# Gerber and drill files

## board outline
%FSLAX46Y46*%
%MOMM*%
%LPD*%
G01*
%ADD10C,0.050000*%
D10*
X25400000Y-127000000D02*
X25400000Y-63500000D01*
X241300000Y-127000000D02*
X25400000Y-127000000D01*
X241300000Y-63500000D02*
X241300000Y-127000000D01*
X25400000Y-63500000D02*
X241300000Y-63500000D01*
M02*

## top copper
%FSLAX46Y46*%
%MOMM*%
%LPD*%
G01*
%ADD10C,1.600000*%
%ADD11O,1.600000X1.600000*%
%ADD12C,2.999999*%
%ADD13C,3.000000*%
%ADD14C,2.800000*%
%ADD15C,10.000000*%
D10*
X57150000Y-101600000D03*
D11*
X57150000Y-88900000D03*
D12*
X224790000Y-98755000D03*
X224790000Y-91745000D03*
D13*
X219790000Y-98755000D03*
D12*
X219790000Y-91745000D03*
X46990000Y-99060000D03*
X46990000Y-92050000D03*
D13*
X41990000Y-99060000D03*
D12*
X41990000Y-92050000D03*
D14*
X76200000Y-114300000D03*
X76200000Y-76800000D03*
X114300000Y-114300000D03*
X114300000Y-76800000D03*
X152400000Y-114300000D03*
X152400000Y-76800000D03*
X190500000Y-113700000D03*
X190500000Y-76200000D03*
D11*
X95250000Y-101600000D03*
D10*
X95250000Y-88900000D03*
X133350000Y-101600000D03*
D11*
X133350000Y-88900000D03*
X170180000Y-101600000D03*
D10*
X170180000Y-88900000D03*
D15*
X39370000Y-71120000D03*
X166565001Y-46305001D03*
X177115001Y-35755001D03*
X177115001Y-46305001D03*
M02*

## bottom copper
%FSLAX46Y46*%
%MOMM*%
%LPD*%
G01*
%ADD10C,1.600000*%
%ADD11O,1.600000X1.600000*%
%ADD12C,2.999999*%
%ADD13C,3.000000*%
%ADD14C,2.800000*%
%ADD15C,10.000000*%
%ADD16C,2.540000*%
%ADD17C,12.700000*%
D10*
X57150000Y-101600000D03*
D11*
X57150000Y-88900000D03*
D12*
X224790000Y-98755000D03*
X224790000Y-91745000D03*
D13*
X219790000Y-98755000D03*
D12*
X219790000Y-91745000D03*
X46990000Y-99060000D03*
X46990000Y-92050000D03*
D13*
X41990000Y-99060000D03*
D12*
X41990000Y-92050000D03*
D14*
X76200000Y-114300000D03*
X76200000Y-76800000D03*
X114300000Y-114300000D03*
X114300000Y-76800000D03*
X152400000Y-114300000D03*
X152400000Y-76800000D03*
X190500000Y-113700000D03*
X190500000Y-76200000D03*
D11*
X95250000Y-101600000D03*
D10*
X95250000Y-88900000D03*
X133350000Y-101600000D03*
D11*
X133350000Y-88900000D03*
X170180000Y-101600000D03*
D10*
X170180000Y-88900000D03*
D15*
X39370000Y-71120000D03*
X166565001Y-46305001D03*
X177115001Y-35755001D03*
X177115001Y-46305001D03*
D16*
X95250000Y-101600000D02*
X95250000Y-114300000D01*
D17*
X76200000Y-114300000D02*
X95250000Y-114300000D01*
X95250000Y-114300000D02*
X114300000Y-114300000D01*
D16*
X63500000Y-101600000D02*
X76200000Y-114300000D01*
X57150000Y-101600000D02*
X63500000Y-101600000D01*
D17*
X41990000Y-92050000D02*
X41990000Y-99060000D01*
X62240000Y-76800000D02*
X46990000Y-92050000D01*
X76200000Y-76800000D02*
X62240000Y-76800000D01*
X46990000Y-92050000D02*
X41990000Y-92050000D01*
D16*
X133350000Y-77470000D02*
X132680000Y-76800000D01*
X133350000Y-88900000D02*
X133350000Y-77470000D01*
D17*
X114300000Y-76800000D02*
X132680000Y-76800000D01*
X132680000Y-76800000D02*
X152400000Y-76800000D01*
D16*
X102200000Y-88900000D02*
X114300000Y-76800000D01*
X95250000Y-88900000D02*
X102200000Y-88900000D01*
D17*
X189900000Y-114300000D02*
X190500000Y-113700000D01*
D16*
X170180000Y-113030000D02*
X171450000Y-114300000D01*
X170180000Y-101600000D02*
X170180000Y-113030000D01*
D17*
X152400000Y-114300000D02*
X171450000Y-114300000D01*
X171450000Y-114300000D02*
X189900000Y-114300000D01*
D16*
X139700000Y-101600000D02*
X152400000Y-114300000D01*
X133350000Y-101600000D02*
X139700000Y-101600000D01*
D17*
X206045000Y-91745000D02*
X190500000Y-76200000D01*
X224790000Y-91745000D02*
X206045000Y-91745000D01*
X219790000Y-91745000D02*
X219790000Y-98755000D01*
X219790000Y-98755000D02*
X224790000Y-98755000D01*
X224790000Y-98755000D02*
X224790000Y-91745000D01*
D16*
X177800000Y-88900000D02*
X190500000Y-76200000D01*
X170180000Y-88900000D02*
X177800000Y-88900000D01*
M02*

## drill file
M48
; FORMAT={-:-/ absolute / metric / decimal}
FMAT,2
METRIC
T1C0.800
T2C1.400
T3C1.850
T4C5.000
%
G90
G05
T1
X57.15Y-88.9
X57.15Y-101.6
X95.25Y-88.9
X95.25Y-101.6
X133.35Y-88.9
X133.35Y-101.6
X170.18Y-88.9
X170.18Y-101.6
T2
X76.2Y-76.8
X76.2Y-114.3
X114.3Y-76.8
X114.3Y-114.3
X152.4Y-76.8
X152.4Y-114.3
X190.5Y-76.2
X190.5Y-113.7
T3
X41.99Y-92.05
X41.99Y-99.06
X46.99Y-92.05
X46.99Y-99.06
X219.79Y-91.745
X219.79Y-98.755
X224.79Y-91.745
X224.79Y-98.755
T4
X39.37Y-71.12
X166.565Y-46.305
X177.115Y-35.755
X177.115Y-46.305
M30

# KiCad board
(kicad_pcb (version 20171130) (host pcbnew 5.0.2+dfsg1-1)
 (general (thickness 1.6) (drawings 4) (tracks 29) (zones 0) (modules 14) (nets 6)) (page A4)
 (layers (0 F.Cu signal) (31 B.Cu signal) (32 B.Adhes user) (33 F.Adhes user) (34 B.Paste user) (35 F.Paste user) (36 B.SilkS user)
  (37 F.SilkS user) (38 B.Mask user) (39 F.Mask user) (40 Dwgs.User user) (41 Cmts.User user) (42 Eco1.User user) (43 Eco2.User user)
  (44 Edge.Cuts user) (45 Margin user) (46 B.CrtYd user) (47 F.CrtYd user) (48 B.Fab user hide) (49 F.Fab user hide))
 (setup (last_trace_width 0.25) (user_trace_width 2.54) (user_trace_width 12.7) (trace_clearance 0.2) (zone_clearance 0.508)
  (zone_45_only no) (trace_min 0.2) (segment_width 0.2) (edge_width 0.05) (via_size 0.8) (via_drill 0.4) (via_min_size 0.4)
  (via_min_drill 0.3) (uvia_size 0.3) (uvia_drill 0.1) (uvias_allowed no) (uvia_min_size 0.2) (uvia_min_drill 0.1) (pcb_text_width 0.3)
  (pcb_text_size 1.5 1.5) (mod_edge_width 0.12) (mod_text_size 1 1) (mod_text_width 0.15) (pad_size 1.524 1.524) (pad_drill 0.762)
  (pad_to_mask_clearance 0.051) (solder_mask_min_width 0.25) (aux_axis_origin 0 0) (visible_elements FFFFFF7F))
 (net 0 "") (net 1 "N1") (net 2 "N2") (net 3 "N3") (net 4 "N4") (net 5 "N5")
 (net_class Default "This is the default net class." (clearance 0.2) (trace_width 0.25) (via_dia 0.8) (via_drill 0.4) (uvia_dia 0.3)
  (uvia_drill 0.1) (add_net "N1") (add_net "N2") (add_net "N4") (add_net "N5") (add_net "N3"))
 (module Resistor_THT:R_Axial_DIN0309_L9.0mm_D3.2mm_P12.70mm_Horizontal (layer F.Cu) (at 57.15 101.6 90)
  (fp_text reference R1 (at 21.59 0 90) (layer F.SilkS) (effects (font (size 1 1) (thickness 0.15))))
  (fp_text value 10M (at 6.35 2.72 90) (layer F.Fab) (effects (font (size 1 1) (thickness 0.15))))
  (pad 1 thru_hole circle (at 0 0 90) (size 1.6 1.6) (drill 0.8) (layers *.Cu *.Mask) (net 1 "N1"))
  (pad 2 thru_hole oval (at 12.7 0 90) (size 1.6 1.6) (drill 0.8) (layers *.Cu *.Mask) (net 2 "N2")))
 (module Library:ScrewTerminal (layer F.Cu) (at 222.29 95.25)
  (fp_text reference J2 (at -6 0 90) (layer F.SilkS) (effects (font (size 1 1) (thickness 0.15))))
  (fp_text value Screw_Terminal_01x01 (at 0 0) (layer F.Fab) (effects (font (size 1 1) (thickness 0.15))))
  (pad 1 thru_hole circle (at 2.5 3.505) (size 2.999999 2.999999) (drill 1.85) (layers *.Cu *.Mask) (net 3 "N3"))
  (pad 1 thru_hole circle (at 2.5 -3.505) (size 2.999999 2.999999) (drill 1.85) (layers *.Cu *.Mask) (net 3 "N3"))
  (pad 1 thru_hole circle (at -2.5 3.505) (size 3 3) (drill 1.85) (layers *.Cu *.Mask) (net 3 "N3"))
  (pad 1 thru_hole circle (at -2.5 -3.505) (size 2.999999 2.999999) (drill 1.85) (layers *.Cu *.Mask) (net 3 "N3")))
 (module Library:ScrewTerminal (layer F.Cu) (at 44.49 95.555)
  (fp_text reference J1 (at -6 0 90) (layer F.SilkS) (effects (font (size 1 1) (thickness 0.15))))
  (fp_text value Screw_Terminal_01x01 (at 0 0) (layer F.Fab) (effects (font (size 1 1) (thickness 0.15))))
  (pad 1 thru_hole circle (at 2.5 3.505) (size 2.999999 2.999999) (drill 1.85) (layers *.Cu *.Mask) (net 2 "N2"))
  (pad 1 thru_hole circle (at 2.5 -3.505) (size 2.999999 2.999999) (drill 1.85) (layers *.Cu *.Mask) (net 2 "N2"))
  (pad 1 thru_hole circle (at -2.5 3.505) (size 3 3) (drill 1.85) (layers *.Cu *.Mask) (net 2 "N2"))
  (pad 1 thru_hole circle (at -2.5 -3.505) (size 2.999999 2.999999) (drill 1.85) (layers *.Cu *.Mask) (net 2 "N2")))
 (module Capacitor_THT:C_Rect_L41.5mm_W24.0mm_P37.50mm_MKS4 (layer F.Cu) (at 76.2 114.3 90)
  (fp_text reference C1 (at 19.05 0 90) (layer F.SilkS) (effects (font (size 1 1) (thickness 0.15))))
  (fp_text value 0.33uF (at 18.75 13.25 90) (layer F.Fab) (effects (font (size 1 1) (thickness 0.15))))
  (pad 1 thru_hole circle (at 0 0 90) (size 2.8 2.8) (drill 1.4) (layers *.Cu *.Mask) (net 1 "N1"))
  (pad 2 thru_hole circle (at 37.5 0 90) (size 2.8 2.8) (drill 1.4) (layers *.Cu *.Mask) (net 2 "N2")))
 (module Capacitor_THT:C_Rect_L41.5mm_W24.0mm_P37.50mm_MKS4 (layer F.Cu) (at 114.3 76.8 270)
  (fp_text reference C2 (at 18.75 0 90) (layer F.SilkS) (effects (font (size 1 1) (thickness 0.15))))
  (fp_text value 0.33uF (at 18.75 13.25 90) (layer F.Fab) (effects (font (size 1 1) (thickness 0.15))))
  (pad 2 thru_hole circle (at 37.5 0 270) (size 2.8 2.8) (drill 1.4) (layers *.Cu *.Mask) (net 1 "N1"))
  (pad 1 thru_hole circle (at 0 0 270) (size 2.8 2.8) (drill 1.4) (layers *.Cu *.Mask) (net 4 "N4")))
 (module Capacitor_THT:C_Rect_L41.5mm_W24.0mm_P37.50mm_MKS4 (layer F.Cu) (at 152.4 114.3 90)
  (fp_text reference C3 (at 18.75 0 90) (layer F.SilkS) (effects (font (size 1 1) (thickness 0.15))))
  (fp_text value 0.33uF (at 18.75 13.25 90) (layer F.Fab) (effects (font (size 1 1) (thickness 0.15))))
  (pad 1 thru_hole circle (at 0 0 90) (size 2.8 2.8) (drill 1.4) (layers *.Cu *.Mask) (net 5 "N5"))
  (pad 2 thru_hole circle (at 37.5 0 90) (size 2.8 2.8) (drill 1.4) (layers *.Cu *.Mask) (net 4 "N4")))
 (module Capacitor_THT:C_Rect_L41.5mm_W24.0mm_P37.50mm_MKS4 (layer F.Cu) (at 190.5 76.2 270)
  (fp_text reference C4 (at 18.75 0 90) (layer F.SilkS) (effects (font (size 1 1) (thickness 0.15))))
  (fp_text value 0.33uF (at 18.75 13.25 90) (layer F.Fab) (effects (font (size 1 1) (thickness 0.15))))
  (pad 2 thru_hole circle (at 37.5 0 270) (size 2.8 2.8) (drill 1.4) (layers *.Cu *.Mask) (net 5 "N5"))
  (pad 1 thru_hole circle (at 0 0 270) (size 2.8 2.8) (drill 1.4) (layers *.Cu *.Mask) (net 3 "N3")))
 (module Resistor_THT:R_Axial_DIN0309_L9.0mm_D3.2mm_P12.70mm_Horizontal (layer F.Cu) (at 95.25 88.9 270)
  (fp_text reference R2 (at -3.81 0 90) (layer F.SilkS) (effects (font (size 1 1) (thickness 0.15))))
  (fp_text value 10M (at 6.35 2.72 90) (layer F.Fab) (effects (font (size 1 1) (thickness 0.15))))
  (pad 2 thru_hole oval (at 12.7 0 270) (size 1.6 1.6) (drill 0.8) (layers *.Cu *.Mask) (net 1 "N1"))
  (pad 1 thru_hole circle (at 0 0 270) (size 1.6 1.6) (drill 0.8) (layers *.Cu *.Mask) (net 4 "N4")))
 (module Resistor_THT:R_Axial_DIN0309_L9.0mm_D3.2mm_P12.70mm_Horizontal (layer F.Cu) (at 133.35 101.6 90)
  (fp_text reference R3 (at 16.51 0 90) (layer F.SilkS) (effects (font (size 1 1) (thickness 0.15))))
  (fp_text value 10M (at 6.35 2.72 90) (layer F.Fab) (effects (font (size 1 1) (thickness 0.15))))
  (pad 1 thru_hole circle (at 0 0 90) (size 1.6 1.6) (drill 0.8) (layers *.Cu *.Mask) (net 5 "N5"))
  (pad 2 thru_hole oval (at 12.7 0 90) (size 1.6 1.6) (drill 0.8) (layers *.Cu *.Mask) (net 4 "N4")))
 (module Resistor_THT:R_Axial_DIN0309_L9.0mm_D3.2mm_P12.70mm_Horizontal (layer F.Cu) (at 170.18 88.9 270)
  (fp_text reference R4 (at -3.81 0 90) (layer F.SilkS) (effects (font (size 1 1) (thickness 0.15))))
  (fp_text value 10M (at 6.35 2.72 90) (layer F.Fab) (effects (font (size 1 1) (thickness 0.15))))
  (pad 2 thru_hole oval (at 12.7 0 270) (size 1.6 1.6) (drill 0.8) (layers *.Cu *.Mask) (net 5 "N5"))
  (pad 1 thru_hole circle (at 0 0 270) (size 1.6 1.6) (drill 0.8) (layers *.Cu *.Mask) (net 3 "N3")))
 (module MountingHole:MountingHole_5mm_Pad (layer F.Cu) (at 39.37 71.12)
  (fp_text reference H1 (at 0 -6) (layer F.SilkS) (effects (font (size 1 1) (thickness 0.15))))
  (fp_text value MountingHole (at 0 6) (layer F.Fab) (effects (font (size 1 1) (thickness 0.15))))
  (pad 1 thru_hole circle (at 0 0) (size 10 10) (drill 5) (layers *.Cu *.Mask)))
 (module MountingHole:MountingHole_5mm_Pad (layer F.Cu) (at 166.565001 46.305001)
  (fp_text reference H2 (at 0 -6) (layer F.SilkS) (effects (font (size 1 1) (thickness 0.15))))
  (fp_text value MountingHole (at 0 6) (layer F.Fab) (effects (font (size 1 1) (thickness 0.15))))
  (pad 1 thru_hole circle (at 0 0) (size 10 10) (drill 5) (layers *.Cu *.Mask)))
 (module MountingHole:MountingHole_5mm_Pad (layer F.Cu) (at 177.115001 35.755001)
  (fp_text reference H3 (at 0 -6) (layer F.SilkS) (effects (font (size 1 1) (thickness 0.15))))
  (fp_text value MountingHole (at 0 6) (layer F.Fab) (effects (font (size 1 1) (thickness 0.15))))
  (pad 1 thru_hole circle (at 0 0) (size 10 10) (drill 5) (layers *.Cu *.Mask)))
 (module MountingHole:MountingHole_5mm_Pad (layer F.Cu) (at 177.115001 46.305001)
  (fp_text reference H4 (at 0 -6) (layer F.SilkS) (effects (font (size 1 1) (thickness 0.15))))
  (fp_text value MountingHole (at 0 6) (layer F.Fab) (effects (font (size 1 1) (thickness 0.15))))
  (pad 1 thru_hole circle (at 0 0) (size 10 10) (drill 5) (layers *.Cu *.Mask)))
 (gr_line (start 25.4 127) (end 25.4 63.5) (layer Edge.Cuts) (width 0.05))
 (gr_line (start 241.3 127) (end 25.4 127) (layer Edge.Cuts) (width 0.05))
 (gr_line (start 241.3 63.5) (end 241.3 127) (layer Edge.Cuts) (width 0.05))
 (gr_line (start 25.4 63.5) (end 241.3 63.5) (layer Edge.Cuts) (width 0.05))
 (segment (start 95.25 101.6) (end 95.25 114.3) (width 2.54) (layer B.Cu) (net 1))
 (segment (start 76.2 114.3) (end 95.25 114.3) (width 12.7) (layer B.Cu) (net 1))
 (segment (start 95.25 114.3) (end 114.3 114.3) (width 12.7) (layer B.Cu) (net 1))
 (segment (start 63.5 101.6) (end 76.2 114.3) (width 2.54) (layer B.Cu) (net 1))
 (segment (start 57.15 101.6) (end 63.5 101.6) (width 2.54) (layer B.Cu) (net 1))
 (segment (start 41.99 92.05) (end 41.99 99.06) (width 12.7) (layer B.Cu) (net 2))
 (segment (start 62.24 76.8) (end 46.99 92.05) (width 12.7) (layer B.Cu) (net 2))
 (segment (start 76.2 76.8) (end 62.24 76.8) (width 12.7) (layer B.Cu) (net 2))
 (segment (start 46.99 92.05) (end 41.99 92.05) (width 12.7) (layer B.Cu) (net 2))
 (segment (start 133.35 77.47) (end 132.68 76.8) (width 2.54) (layer B.Cu) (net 4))
 (segment (start 133.35 88.9) (end 133.35 77.47) (width 2.54) (layer B.Cu) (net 4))
 (segment (start 114.3 76.8) (end 132.68 76.8) (width 12.7) (layer B.Cu) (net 4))
 (segment (start 132.68 76.8) (end 152.4 76.8) (width 12.7) (layer B.Cu) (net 4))
 (segment (start 102.2 88.9) (end 114.3 76.8) (width 2.54) (layer B.Cu) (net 4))
 (segment (start 95.25 88.9) (end 102.2 88.9) (width 2.54) (layer B.Cu) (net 4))
 (segment (start 189.9 114.3) (end 190.5 113.7) (width 12.7) (layer B.Cu) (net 5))
 (segment (start 170.18 113.03) (end 171.45 114.3) (width 2.54) (layer B.Cu) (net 5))
 (segment (start 170.18 101.6) (end 170.18 113.03) (width 2.54) (layer B.Cu) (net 5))
 (segment (start 152.4 114.3) (end 171.45 114.3) (width 12.7) (layer B.Cu) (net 5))
 (segment (start 171.45 114.3) (end 189.9 114.3) (width 12.7) (layer B.Cu) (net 5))
 (segment (start 139.7 101.6) (end 152.4 114.3) (width 2.54) (layer B.Cu) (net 5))
 (segment (start 133.35 101.6) (end 139.7 101.6) (width 2.54) (layer B.Cu) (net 5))
 (segment (start 206.045 91.745) (end 190.5 76.2) (width 12.7) (layer B.Cu) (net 3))
 (segment (start 224.79 91.745) (end 206.045 91.745) (width 12.7) (layer B.Cu) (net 3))
 (segment (start 219.79 91.745) (end 219.79 98.755) (width 12.7) (layer B.Cu) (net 3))
 (segment (start 219.79 98.755) (end 224.79 98.755) (width 12.7) (layer B.Cu) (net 3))
 (segment (start 224.79 98.755) (end 224.79 91.745) (width 12.7) (layer B.Cu) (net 3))
 (segment (start 177.8 88.9) (end 190.5 76.2) (width 2.54) (layer B.Cu) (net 3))
 (segment (start 170.18 88.9) (end 177.8 88.9) (width 2.54) (layer B.Cu) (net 3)))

